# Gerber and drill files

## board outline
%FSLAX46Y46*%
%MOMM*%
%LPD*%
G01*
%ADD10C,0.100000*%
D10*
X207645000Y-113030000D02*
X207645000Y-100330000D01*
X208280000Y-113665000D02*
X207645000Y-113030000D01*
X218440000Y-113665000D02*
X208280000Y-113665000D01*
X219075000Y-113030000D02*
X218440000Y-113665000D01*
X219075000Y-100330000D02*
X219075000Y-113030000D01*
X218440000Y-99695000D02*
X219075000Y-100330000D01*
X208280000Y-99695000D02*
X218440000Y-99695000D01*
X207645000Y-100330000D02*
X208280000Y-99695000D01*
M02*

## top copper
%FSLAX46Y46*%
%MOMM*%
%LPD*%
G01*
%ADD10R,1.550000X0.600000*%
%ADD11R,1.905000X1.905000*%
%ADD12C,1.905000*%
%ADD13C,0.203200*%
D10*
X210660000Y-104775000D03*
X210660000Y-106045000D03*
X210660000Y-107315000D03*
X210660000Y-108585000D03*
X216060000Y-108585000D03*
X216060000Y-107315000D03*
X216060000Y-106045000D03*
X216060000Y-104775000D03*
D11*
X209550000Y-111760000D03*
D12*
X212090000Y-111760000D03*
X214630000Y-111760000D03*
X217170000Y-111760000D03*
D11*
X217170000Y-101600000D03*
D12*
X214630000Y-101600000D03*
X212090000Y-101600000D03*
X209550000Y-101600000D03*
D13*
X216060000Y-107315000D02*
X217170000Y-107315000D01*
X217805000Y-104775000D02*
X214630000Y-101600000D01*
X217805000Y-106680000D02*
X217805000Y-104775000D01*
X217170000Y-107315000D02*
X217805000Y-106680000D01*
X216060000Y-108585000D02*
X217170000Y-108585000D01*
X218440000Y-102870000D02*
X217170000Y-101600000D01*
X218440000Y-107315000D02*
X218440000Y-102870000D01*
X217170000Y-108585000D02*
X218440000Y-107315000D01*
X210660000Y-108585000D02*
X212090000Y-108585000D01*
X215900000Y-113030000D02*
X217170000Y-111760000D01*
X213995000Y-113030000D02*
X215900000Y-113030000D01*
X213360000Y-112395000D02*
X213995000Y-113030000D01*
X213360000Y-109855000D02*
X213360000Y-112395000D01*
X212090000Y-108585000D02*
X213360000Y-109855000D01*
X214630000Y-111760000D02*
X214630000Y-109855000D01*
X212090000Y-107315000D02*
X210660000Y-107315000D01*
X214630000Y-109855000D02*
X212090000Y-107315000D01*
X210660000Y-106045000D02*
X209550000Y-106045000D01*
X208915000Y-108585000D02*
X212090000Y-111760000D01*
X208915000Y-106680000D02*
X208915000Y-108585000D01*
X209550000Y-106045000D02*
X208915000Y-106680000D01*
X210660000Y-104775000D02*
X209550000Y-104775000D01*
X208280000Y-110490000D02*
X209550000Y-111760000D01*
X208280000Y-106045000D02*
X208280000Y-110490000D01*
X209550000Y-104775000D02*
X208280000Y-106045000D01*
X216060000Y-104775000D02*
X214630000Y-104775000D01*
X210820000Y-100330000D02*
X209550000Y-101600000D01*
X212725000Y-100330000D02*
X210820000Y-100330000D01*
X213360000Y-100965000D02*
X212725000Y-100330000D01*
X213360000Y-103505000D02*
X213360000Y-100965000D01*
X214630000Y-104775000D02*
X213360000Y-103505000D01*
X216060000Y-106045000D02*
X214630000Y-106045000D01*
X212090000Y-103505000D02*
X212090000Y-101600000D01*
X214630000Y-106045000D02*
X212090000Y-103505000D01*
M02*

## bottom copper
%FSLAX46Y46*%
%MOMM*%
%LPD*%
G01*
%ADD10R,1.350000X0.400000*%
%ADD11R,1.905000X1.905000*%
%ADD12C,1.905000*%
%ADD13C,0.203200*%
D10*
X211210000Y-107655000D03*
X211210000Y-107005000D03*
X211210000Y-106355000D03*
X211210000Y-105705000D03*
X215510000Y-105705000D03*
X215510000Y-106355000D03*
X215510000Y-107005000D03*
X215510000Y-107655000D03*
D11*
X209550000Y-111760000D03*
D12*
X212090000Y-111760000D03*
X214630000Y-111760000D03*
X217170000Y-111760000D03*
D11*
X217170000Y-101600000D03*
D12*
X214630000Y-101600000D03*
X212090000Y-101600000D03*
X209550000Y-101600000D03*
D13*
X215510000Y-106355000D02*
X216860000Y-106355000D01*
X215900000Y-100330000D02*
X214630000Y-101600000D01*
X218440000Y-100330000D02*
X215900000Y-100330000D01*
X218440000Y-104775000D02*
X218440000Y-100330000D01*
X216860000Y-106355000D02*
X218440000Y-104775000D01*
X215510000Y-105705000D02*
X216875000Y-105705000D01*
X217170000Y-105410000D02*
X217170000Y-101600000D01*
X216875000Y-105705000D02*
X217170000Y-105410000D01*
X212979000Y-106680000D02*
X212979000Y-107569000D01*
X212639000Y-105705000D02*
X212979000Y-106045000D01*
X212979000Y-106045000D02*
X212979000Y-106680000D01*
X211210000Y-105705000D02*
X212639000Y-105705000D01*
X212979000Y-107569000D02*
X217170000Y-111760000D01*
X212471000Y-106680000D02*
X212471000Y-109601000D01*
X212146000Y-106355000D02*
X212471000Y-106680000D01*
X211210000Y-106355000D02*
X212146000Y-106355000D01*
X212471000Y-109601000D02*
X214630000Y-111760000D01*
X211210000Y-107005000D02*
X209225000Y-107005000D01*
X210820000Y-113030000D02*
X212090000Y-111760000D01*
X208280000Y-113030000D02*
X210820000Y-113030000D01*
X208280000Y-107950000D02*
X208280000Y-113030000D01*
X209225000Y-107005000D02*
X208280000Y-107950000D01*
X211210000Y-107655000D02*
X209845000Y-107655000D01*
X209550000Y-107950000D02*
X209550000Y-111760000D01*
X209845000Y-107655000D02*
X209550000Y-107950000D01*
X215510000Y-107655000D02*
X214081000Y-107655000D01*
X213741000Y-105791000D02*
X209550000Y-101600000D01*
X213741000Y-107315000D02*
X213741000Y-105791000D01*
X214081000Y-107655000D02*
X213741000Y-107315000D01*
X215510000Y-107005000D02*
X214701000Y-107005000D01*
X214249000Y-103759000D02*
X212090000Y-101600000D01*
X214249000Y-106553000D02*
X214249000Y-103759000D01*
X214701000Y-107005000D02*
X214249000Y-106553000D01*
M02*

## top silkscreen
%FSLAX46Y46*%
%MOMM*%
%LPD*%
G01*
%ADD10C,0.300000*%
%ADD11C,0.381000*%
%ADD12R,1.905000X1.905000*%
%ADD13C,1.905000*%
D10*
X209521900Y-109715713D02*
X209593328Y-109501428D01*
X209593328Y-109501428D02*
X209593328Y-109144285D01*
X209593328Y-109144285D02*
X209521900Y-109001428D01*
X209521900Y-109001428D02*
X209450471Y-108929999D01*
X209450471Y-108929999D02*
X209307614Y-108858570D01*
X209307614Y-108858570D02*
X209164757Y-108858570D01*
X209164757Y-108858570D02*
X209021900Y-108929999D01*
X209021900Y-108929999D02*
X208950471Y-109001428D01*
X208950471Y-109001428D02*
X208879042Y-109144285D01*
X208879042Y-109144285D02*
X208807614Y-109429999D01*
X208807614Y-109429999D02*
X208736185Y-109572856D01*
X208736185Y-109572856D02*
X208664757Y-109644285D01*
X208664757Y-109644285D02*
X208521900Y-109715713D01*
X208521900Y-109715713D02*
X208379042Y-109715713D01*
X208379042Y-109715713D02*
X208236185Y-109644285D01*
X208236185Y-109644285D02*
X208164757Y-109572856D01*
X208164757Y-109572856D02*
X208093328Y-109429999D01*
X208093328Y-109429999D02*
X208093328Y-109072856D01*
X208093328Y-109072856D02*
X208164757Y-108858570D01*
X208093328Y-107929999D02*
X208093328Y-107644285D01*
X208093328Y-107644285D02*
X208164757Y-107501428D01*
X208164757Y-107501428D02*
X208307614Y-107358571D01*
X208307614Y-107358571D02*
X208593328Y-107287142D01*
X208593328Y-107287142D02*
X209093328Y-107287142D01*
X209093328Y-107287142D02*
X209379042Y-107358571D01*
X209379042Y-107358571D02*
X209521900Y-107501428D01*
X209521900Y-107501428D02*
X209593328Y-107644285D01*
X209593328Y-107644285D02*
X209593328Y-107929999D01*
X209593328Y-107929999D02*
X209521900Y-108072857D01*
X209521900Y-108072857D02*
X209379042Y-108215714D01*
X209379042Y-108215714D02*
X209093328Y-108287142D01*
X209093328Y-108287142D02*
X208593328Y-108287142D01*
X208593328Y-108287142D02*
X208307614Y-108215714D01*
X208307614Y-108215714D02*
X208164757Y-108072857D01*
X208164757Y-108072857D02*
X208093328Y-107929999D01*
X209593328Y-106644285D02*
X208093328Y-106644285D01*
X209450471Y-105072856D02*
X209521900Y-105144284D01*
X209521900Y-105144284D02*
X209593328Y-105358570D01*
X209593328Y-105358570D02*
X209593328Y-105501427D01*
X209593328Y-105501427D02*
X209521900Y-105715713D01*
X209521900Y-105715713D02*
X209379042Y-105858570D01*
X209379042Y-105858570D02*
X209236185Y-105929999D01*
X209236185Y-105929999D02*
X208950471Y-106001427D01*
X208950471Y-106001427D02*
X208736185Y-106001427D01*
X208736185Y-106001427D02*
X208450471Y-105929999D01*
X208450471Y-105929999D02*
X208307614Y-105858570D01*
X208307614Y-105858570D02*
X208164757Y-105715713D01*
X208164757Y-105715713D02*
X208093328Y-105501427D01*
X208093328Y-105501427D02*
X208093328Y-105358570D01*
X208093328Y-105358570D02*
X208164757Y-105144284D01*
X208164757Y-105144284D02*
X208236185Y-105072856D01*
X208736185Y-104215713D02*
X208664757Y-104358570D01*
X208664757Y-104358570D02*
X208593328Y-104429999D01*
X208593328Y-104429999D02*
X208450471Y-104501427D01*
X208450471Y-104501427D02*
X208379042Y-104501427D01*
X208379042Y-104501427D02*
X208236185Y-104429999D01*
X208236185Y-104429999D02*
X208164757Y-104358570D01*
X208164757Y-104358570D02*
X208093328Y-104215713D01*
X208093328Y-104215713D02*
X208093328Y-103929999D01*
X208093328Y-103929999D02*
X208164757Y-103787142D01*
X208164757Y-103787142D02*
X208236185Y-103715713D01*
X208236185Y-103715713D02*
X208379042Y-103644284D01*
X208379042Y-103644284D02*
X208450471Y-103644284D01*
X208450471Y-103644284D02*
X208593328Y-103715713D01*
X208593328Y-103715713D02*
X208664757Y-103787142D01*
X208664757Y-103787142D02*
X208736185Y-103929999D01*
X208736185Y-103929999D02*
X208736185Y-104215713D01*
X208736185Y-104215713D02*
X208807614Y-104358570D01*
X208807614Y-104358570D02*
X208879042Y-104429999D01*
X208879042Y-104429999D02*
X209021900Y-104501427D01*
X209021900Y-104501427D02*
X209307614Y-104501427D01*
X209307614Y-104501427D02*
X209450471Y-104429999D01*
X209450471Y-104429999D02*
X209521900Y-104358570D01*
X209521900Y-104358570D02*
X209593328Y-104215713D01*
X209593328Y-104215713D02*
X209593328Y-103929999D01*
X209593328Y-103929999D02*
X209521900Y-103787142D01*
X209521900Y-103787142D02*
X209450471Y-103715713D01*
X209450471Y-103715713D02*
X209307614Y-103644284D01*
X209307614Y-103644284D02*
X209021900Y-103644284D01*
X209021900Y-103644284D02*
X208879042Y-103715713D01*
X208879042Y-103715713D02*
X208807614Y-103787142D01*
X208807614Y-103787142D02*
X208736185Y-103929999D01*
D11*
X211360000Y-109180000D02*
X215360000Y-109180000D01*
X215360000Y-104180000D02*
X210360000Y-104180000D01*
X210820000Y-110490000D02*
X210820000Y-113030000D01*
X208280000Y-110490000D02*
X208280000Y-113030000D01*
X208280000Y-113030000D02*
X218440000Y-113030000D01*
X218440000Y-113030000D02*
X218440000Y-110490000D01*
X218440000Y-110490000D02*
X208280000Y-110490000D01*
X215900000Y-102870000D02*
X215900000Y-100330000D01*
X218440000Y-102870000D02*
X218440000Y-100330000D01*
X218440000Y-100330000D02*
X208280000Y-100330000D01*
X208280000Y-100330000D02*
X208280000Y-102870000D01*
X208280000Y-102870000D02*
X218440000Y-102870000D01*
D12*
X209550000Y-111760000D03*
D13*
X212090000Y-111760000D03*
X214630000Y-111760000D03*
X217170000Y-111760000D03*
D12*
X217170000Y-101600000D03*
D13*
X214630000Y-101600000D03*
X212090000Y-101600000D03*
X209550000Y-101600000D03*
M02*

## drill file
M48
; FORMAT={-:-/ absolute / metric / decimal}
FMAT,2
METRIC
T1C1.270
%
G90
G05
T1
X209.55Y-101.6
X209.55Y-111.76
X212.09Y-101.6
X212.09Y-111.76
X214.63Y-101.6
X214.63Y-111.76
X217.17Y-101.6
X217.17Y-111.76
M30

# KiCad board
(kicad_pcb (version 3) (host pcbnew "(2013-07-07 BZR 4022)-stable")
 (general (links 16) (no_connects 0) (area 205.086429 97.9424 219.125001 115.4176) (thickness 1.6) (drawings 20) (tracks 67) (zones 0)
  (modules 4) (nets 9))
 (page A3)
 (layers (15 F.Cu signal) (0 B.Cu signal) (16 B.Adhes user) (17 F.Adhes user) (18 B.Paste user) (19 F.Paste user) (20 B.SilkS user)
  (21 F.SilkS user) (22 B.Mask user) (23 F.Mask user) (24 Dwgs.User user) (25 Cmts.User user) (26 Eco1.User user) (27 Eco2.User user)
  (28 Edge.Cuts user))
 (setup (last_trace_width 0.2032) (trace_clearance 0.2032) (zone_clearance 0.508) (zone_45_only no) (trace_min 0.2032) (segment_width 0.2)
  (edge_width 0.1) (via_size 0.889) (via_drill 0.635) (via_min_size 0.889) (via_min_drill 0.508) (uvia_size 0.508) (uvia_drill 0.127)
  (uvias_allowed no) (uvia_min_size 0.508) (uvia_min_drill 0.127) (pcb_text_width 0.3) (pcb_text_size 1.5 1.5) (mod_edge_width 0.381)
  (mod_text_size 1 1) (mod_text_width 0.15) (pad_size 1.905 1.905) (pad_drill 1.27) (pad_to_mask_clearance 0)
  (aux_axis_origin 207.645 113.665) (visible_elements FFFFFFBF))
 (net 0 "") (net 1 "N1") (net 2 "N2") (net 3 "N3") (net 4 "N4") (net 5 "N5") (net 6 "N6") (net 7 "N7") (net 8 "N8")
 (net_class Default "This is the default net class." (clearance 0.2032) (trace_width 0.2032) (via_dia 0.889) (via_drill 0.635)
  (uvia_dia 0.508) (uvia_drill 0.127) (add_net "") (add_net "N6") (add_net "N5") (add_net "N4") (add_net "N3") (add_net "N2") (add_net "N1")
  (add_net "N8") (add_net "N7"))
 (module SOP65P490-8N (layer B.Cu) (at 213.36 106.68 90)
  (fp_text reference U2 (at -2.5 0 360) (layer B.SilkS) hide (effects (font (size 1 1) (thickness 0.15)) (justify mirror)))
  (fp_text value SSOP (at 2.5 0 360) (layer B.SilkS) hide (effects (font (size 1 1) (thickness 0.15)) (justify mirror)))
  (pad 1 smd rect (at -0.975 -2.15 90) (size 0.4 1.35) (layers B.Cu B.Paste B.Mask) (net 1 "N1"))
  (pad 2 smd rect (at -0.325 -2.15 90) (size 0.4 1.35) (layers B.Cu B.Paste B.Mask) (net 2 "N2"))
  (pad 3 smd rect (at 0.325 -2.15 90) (size 0.4 1.35) (layers B.Cu B.Paste B.Mask) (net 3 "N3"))
  (pad 4 smd rect (at 0.975 -2.15 90) (size 0.4 1.35) (layers B.Cu B.Paste B.Mask) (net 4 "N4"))
  (pad 5 smd rect (at 0.975 2.15 90) (size 0.4 1.35) (layers B.Cu B.Paste B.Mask) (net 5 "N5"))
  (pad 6 smd rect (at 0.325 2.15 90) (size 0.4 1.35) (layers B.Cu B.Paste B.Mask) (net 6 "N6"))
  (pad 7 smd rect (at -0.325 2.15 90) (size 0.4 1.35) (layers B.Cu B.Paste B.Mask) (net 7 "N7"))
  (pad 8 smd rect (at -0.975 2.15 90) (size 0.4 1.35) (layers B.Cu B.Paste B.Mask) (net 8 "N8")))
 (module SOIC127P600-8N (layer F.Cu) (at 213.36 106.68 270)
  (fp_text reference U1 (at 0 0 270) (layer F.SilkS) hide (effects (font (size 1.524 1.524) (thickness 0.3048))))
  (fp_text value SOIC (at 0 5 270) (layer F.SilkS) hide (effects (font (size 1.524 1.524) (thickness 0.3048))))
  (fp_line (start 2.5 2) (end 2.5 -2) (layer F.SilkS) (width 0.381))
  (fp_line (start -2.5 -2) (end -2.5 3) (layer F.SilkS) (width 0.381))
  (pad 1 smd rect (at -1.905 2.7 270) (size 0.6 1.55) (layers F.Cu F.Paste F.Mask) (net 1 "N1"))
  (pad 2 smd rect (at -0.635 2.7 270) (size 0.6 1.55) (layers F.Cu F.Paste F.Mask) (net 2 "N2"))
  (pad 3 smd rect (at 0.635 2.7 270) (size 0.6 1.55) (layers F.Cu F.Paste F.Mask) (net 3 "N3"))
  (pad 4 smd rect (at 1.905 2.7 270) (size 0.6 1.55) (layers F.Cu F.Paste F.Mask) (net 4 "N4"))
  (pad 5 smd rect (at 1.905 -2.7 270) (size 0.6 1.55) (layers F.Cu F.Paste F.Mask) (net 5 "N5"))
  (pad 6 smd rect (at 0.635 -2.7 270) (size 0.6 1.55) (layers F.Cu F.Paste F.Mask) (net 6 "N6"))
  (pad 7 smd rect (at -0.635 -2.7 270) (size 0.6 1.55) (layers F.Cu F.Paste F.Mask) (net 7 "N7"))
  (pad 8 smd rect (at -1.905 -2.7 270) (size 0.6 1.55) (layers F.Cu F.Paste F.Mask) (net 8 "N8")))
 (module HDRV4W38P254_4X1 (layer F.Cu) (at 213.36 111.76)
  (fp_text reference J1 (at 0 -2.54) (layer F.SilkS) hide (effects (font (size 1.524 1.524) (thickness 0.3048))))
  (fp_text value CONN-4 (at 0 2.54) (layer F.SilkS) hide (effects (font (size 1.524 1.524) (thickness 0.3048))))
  (fp_line (start -2.54 -1.27) (end -2.54 1.27) (layer F.SilkS) (width 0.381))
  (fp_line (start -5.08 -1.27) (end -5.08 1.27) (layer F.SilkS) (width 0.381))
  (fp_line (start -5.08 1.27) (end 5.08 1.27) (layer F.SilkS) (width 0.381))
  (fp_line (start 5.08 1.27) (end 5.08 -1.27) (layer F.SilkS) (width 0.381))
  (fp_line (start 5.08 -1.27) (end -5.08 -1.27) (layer F.SilkS) (width 0.381))
  (pad 1 thru_hole rect (at -3.81 0) (size 1.905 1.905) (drill 1.27) (layers *.Cu *.Mask F.SilkS) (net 1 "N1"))
  (pad 2 thru_hole circle (at -1.27 0) (size 1.905 1.905) (drill 1.27) (layers *.Cu *.Mask F.SilkS) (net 2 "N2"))
  (pad 3 thru_hole circle (at 1.27 0) (size 1.905 1.905) (drill 1.27) (layers *.Cu *.Mask F.SilkS) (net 3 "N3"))
  (pad 4 thru_hole circle (at 3.81 0) (size 1.905 1.905) (drill 1.27) (layers *.Cu *.Mask F.SilkS) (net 4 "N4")))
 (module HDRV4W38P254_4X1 (layer F.Cu) (at 213.36 101.6 180)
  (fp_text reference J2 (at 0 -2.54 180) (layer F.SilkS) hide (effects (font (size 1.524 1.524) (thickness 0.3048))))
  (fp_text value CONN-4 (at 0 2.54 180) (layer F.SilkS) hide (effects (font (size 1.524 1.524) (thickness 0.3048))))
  (fp_line (start -2.54 -1.27) (end -2.54 1.27) (layer F.SilkS) (width 0.381))
  (fp_line (start -5.08 -1.27) (end -5.08 1.27) (layer F.SilkS) (width 0.381))
  (fp_line (start -5.08 1.27) (end 5.08 1.27) (layer F.SilkS) (width 0.381))
  (fp_line (start 5.08 1.27) (end 5.08 -1.27) (layer F.SilkS) (width 0.381))
  (fp_line (start 5.08 -1.27) (end -5.08 -1.27) (layer F.SilkS) (width 0.381))
  (pad 1 thru_hole rect (at -3.81 0 180) (size 1.905 1.905) (drill 1.27) (layers *.Cu *.Mask F.SilkS) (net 5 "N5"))
  (pad 2 thru_hole circle (at -1.27 0 180) (size 1.905 1.905) (drill 1.27) (layers *.Cu *.Mask F.SilkS) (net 6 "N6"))
  (pad 3 thru_hole circle (at 1.27 0 180) (size 1.905 1.905) (drill 1.27) (layers *.Cu *.Mask F.SilkS) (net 7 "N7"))
  (pad 4 thru_hole circle (at 3.81 0 180) (size 1.905 1.905) (drill 1.27) (layers *.Cu *.Mask F.SilkS) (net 8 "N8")))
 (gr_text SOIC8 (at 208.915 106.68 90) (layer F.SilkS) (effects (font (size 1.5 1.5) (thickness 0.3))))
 (gr_line (start 207.645 113.03) (end 207.645 100.33) (angle 90) (layer Edge.Cuts) (width 0.1))
 (gr_line (start 208.28 113.665) (end 207.645 113.03) (angle 90) (layer Edge.Cuts) (width 0.1))
 (gr_line (start 218.44 113.665) (end 208.28 113.665) (angle 90) (layer Edge.Cuts) (width 0.1))
 (gr_line (start 219.075 113.03) (end 218.44 113.665) (angle 90) (layer Edge.Cuts) (width 0.1))
 (gr_line (start 219.075 100.33) (end 219.075 113.03) (angle 90) (layer Edge.Cuts) (width 0.1))
 (gr_line (start 218.44 99.695) (end 219.075 100.33) (angle 90) (layer Edge.Cuts) (width 0.1))
 (gr_line (start 208.28 99.695) (end 218.44 99.695) (angle 90) (layer Edge.Cuts) (width 0.1))
 (gr_line (start 207.645 100.33) (end 208.28 99.695) (angle 90) (layer Edge.Cuts) (width 0.1))
 (segment (start 215.51 106.355) (end 216.86 106.355) (width 0.2032) (layer B.Cu) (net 6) (status 400000))
 (segment (start 215.9 100.33) (end 214.63 101.6) (width 0.2032) (layer B.Cu) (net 6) (status 800000))
 (segment (start 218.44 100.33) (end 215.9 100.33) (width 0.2032) (layer B.Cu) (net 6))
 (segment (start 218.44 104.775) (end 218.44 100.33) (width 0.2032) (layer B.Cu) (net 6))
 (segment (start 216.86 106.355) (end 218.44 104.775) (width 0.2032) (layer B.Cu) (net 6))
 (segment (start 216.06 107.315) (end 217.17 107.315) (width 0.2032) (layer F.Cu) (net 6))
 (segment (start 217.805 104.775) (end 214.63 101.6) (width 0.2032) (layer F.Cu) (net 6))
 (segment (start 217.805 106.68) (end 217.805 104.775) (width 0.2032) (layer F.Cu) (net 6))
 (segment (start 217.17 107.315) (end 217.805 106.68) (width 0.2032) (layer F.Cu) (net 6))
 (segment (start 215.51 105.705) (end 216.875 105.705) (width 0.2032) (layer B.Cu) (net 5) (status 400000))
 (segment (start 217.17 105.41) (end 217.17 101.6) (width 0.2032) (layer B.Cu) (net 5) (status 800000))
 (segment (start 216.875 105.705) (end 217.17 105.41) (width 0.2032) (layer B.Cu) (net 5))
 (segment (start 216.06 108.585) (end 217.17 108.585) (width 0.2032) (layer F.Cu) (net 5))
 (segment (start 218.44 102.87) (end 217.17 101.6) (width 0.2032) (layer F.Cu) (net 5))
 (segment (start 218.44 107.315) (end 218.44 102.87) (width 0.2032) (layer F.Cu) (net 5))
 (segment (start 217.17 108.585) (end 218.44 107.315) (width 0.2032) (layer F.Cu) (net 5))
 (segment (start 212.979 106.68) (end 212.979 107.569) (width 0.2032) (layer B.Cu) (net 4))
 (segment (start 212.639 105.705) (end 212.979 106.045) (width 0.2032) (layer B.Cu) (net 4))
 (segment (start 212.979 106.045) (end 212.979 106.68) (width 0.2032) (layer B.Cu) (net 4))
 (segment (start 211.21 105.705) (end 212.639 105.705) (width 0.2032) (layer B.Cu) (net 4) (status 400000))
 (segment (start 212.979 107.569) (end 217.17 111.76) (width 0.2032) (layer B.Cu) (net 4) (status 800000))
 (segment (start 210.66 108.585) (end 212.09 108.585) (width 0.2032) (layer F.Cu) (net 4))
 (segment (start 215.9 113.03) (end 217.17 111.76) (width 0.2032) (layer F.Cu) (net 4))
 (segment (start 213.995 113.03) (end 215.9 113.03) (width 0.2032) (layer F.Cu) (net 4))
 (segment (start 213.36 112.395) (end 213.995 113.03) (width 0.2032) (layer F.Cu) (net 4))
 (segment (start 213.36 109.855) (end 213.36 112.395) (width 0.2032) (layer F.Cu) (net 4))
 (segment (start 212.09 108.585) (end 213.36 109.855) (width 0.2032) (layer F.Cu) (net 4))
 (segment (start 212.471 106.68) (end 212.471 109.601) (width 0.2032) (layer B.Cu) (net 3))
 (segment (start 212.146 106.355) (end 212.471 106.68) (width 0.2032) (layer B.Cu) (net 3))
 (segment (start 211.21 106.355) (end 212.146 106.355) (width 0.2032) (layer B.Cu) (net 3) (status 400000))
 (segment (start 212.471 109.601) (end 214.63 111.76) (width 0.2032) (layer B.Cu) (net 3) (status 800000))
 (segment (start 214.63 111.76) (end 214.63 109.855) (width 0.2032) (layer F.Cu) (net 3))
 (segment (start 212.09 107.315) (end 210.66 107.315) (width 0.2032) (layer F.Cu) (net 3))
 (segment (start 214.63 109.855) (end 212.09 107.315) (width 0.2032) (layer F.Cu) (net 3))
 (segment (start 211.21 107.005) (end 209.225 107.005) (width 0.2032) (layer B.Cu) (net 2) (status 400000))
 (segment (start 210.82 113.03) (end 212.09 111.76) (width 0.2032) (layer B.Cu) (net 2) (status 800000))
 (segment (start 208.28 113.03) (end 210.82 113.03) (width 0.2032) (layer B.Cu) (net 2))
 (segment (start 208.28 107.95) (end 208.28 113.03) (width 0.2032) (layer B.Cu) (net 2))
 (segment (start 209.225 107.005) (end 208.28 107.95) (width 0.2032) (layer B.Cu) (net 2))
 (segment (start 210.66 106.045) (end 209.55 106.045) (width 0.2032) (layer F.Cu) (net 2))
 (segment (start 208.915 108.585) (end 212.09 111.76) (width 0.2032) (layer F.Cu) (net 2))
 (segment (start 208.915 106.68) (end 208.915 108.585) (width 0.2032) (layer F.Cu) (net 2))
 (segment (start 209.55 106.045) (end 208.915 106.68) (width 0.2032) (layer F.Cu) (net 2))
 (segment (start 211.21 107.655) (end 209.845 107.655) (width 0.2032) (layer B.Cu) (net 1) (status 400000))
 (segment (start 209.55 107.95) (end 209.55 111.76) (width 0.2032) (layer B.Cu) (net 1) (status 800000))
 (segment (start 209.845 107.655) (end 209.55 107.95) (width 0.2032) (layer B.Cu) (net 1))
 (segment (start 210.66 104.775) (end 209.55 104.775) (width 0.2032) (layer F.Cu) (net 1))
 (segment (start 208.28 110.49) (end 209.55 111.76) (width 0.2032) (layer F.Cu) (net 1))
 (segment (start 208.28 106.045) (end 208.28 110.49) (width 0.2032) (layer F.Cu) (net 1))
 (segment (start 209.55 104.775) (end 208.28 106.045) (width 0.2032) (layer F.Cu) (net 1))
 (segment (start 215.51 107.655) (end 214.081 107.655) (width 0.2032) (layer B.Cu) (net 8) (status 400000))
 (segment (start 213.741 105.791) (end 209.55 101.6) (width 0.2032) (layer B.Cu) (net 8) (status 800000))
 (segment (start 213.741 107.315) (end 213.741 105.791) (width 0.2032) (layer B.Cu) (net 8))
 (segment (start 214.081 107.655) (end 213.741 107.315) (width 0.2032) (layer B.Cu) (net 8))
 (segment (start 216.06 104.775) (end 214.63 104.775) (width 0.2032) (layer F.Cu) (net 8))
 (segment (start 210.82 100.33) (end 209.55 101.6) (width 0.2032) (layer F.Cu) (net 8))
 (segment (start 212.725 100.33) (end 210.82 100.33) (width 0.2032) (layer F.Cu) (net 8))
 (segment (start 213.36 100.965) (end 212.725 100.33) (width 0.2032) (layer F.Cu) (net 8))
 (segment (start 213.36 103.505) (end 213.36 100.965) (width 0.2032) (layer F.Cu) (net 8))
 (segment (start 214.63 104.775) (end 213.36 103.505) (width 0.2032) (layer F.Cu) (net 8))
 (segment (start 215.51 107.005) (end 214.701 107.005) (width 0.2032) (layer B.Cu) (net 7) (status 400000))
 (segment (start 214.249 103.759) (end 212.09 101.6) (width 0.2032) (layer B.Cu) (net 7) (status 800000))
 (segment (start 214.249 106.553) (end 214.249 103.759) (width 0.2032) (layer B.Cu) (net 7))
 (segment (start 214.701 107.005) (end 214.249 106.553) (width 0.2032) (layer B.Cu) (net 7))
 (segment (start 216.06 106.045) (end 214.63 106.045) (width 0.2032) (layer F.Cu) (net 7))
 (segment (start 212.09 103.505) (end 212.09 101.6) (width 0.2032) (layer F.Cu) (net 7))
 (segment (start 214.63 106.045) (end 212.09 103.505) (width 0.2032) (layer F.Cu) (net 7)))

